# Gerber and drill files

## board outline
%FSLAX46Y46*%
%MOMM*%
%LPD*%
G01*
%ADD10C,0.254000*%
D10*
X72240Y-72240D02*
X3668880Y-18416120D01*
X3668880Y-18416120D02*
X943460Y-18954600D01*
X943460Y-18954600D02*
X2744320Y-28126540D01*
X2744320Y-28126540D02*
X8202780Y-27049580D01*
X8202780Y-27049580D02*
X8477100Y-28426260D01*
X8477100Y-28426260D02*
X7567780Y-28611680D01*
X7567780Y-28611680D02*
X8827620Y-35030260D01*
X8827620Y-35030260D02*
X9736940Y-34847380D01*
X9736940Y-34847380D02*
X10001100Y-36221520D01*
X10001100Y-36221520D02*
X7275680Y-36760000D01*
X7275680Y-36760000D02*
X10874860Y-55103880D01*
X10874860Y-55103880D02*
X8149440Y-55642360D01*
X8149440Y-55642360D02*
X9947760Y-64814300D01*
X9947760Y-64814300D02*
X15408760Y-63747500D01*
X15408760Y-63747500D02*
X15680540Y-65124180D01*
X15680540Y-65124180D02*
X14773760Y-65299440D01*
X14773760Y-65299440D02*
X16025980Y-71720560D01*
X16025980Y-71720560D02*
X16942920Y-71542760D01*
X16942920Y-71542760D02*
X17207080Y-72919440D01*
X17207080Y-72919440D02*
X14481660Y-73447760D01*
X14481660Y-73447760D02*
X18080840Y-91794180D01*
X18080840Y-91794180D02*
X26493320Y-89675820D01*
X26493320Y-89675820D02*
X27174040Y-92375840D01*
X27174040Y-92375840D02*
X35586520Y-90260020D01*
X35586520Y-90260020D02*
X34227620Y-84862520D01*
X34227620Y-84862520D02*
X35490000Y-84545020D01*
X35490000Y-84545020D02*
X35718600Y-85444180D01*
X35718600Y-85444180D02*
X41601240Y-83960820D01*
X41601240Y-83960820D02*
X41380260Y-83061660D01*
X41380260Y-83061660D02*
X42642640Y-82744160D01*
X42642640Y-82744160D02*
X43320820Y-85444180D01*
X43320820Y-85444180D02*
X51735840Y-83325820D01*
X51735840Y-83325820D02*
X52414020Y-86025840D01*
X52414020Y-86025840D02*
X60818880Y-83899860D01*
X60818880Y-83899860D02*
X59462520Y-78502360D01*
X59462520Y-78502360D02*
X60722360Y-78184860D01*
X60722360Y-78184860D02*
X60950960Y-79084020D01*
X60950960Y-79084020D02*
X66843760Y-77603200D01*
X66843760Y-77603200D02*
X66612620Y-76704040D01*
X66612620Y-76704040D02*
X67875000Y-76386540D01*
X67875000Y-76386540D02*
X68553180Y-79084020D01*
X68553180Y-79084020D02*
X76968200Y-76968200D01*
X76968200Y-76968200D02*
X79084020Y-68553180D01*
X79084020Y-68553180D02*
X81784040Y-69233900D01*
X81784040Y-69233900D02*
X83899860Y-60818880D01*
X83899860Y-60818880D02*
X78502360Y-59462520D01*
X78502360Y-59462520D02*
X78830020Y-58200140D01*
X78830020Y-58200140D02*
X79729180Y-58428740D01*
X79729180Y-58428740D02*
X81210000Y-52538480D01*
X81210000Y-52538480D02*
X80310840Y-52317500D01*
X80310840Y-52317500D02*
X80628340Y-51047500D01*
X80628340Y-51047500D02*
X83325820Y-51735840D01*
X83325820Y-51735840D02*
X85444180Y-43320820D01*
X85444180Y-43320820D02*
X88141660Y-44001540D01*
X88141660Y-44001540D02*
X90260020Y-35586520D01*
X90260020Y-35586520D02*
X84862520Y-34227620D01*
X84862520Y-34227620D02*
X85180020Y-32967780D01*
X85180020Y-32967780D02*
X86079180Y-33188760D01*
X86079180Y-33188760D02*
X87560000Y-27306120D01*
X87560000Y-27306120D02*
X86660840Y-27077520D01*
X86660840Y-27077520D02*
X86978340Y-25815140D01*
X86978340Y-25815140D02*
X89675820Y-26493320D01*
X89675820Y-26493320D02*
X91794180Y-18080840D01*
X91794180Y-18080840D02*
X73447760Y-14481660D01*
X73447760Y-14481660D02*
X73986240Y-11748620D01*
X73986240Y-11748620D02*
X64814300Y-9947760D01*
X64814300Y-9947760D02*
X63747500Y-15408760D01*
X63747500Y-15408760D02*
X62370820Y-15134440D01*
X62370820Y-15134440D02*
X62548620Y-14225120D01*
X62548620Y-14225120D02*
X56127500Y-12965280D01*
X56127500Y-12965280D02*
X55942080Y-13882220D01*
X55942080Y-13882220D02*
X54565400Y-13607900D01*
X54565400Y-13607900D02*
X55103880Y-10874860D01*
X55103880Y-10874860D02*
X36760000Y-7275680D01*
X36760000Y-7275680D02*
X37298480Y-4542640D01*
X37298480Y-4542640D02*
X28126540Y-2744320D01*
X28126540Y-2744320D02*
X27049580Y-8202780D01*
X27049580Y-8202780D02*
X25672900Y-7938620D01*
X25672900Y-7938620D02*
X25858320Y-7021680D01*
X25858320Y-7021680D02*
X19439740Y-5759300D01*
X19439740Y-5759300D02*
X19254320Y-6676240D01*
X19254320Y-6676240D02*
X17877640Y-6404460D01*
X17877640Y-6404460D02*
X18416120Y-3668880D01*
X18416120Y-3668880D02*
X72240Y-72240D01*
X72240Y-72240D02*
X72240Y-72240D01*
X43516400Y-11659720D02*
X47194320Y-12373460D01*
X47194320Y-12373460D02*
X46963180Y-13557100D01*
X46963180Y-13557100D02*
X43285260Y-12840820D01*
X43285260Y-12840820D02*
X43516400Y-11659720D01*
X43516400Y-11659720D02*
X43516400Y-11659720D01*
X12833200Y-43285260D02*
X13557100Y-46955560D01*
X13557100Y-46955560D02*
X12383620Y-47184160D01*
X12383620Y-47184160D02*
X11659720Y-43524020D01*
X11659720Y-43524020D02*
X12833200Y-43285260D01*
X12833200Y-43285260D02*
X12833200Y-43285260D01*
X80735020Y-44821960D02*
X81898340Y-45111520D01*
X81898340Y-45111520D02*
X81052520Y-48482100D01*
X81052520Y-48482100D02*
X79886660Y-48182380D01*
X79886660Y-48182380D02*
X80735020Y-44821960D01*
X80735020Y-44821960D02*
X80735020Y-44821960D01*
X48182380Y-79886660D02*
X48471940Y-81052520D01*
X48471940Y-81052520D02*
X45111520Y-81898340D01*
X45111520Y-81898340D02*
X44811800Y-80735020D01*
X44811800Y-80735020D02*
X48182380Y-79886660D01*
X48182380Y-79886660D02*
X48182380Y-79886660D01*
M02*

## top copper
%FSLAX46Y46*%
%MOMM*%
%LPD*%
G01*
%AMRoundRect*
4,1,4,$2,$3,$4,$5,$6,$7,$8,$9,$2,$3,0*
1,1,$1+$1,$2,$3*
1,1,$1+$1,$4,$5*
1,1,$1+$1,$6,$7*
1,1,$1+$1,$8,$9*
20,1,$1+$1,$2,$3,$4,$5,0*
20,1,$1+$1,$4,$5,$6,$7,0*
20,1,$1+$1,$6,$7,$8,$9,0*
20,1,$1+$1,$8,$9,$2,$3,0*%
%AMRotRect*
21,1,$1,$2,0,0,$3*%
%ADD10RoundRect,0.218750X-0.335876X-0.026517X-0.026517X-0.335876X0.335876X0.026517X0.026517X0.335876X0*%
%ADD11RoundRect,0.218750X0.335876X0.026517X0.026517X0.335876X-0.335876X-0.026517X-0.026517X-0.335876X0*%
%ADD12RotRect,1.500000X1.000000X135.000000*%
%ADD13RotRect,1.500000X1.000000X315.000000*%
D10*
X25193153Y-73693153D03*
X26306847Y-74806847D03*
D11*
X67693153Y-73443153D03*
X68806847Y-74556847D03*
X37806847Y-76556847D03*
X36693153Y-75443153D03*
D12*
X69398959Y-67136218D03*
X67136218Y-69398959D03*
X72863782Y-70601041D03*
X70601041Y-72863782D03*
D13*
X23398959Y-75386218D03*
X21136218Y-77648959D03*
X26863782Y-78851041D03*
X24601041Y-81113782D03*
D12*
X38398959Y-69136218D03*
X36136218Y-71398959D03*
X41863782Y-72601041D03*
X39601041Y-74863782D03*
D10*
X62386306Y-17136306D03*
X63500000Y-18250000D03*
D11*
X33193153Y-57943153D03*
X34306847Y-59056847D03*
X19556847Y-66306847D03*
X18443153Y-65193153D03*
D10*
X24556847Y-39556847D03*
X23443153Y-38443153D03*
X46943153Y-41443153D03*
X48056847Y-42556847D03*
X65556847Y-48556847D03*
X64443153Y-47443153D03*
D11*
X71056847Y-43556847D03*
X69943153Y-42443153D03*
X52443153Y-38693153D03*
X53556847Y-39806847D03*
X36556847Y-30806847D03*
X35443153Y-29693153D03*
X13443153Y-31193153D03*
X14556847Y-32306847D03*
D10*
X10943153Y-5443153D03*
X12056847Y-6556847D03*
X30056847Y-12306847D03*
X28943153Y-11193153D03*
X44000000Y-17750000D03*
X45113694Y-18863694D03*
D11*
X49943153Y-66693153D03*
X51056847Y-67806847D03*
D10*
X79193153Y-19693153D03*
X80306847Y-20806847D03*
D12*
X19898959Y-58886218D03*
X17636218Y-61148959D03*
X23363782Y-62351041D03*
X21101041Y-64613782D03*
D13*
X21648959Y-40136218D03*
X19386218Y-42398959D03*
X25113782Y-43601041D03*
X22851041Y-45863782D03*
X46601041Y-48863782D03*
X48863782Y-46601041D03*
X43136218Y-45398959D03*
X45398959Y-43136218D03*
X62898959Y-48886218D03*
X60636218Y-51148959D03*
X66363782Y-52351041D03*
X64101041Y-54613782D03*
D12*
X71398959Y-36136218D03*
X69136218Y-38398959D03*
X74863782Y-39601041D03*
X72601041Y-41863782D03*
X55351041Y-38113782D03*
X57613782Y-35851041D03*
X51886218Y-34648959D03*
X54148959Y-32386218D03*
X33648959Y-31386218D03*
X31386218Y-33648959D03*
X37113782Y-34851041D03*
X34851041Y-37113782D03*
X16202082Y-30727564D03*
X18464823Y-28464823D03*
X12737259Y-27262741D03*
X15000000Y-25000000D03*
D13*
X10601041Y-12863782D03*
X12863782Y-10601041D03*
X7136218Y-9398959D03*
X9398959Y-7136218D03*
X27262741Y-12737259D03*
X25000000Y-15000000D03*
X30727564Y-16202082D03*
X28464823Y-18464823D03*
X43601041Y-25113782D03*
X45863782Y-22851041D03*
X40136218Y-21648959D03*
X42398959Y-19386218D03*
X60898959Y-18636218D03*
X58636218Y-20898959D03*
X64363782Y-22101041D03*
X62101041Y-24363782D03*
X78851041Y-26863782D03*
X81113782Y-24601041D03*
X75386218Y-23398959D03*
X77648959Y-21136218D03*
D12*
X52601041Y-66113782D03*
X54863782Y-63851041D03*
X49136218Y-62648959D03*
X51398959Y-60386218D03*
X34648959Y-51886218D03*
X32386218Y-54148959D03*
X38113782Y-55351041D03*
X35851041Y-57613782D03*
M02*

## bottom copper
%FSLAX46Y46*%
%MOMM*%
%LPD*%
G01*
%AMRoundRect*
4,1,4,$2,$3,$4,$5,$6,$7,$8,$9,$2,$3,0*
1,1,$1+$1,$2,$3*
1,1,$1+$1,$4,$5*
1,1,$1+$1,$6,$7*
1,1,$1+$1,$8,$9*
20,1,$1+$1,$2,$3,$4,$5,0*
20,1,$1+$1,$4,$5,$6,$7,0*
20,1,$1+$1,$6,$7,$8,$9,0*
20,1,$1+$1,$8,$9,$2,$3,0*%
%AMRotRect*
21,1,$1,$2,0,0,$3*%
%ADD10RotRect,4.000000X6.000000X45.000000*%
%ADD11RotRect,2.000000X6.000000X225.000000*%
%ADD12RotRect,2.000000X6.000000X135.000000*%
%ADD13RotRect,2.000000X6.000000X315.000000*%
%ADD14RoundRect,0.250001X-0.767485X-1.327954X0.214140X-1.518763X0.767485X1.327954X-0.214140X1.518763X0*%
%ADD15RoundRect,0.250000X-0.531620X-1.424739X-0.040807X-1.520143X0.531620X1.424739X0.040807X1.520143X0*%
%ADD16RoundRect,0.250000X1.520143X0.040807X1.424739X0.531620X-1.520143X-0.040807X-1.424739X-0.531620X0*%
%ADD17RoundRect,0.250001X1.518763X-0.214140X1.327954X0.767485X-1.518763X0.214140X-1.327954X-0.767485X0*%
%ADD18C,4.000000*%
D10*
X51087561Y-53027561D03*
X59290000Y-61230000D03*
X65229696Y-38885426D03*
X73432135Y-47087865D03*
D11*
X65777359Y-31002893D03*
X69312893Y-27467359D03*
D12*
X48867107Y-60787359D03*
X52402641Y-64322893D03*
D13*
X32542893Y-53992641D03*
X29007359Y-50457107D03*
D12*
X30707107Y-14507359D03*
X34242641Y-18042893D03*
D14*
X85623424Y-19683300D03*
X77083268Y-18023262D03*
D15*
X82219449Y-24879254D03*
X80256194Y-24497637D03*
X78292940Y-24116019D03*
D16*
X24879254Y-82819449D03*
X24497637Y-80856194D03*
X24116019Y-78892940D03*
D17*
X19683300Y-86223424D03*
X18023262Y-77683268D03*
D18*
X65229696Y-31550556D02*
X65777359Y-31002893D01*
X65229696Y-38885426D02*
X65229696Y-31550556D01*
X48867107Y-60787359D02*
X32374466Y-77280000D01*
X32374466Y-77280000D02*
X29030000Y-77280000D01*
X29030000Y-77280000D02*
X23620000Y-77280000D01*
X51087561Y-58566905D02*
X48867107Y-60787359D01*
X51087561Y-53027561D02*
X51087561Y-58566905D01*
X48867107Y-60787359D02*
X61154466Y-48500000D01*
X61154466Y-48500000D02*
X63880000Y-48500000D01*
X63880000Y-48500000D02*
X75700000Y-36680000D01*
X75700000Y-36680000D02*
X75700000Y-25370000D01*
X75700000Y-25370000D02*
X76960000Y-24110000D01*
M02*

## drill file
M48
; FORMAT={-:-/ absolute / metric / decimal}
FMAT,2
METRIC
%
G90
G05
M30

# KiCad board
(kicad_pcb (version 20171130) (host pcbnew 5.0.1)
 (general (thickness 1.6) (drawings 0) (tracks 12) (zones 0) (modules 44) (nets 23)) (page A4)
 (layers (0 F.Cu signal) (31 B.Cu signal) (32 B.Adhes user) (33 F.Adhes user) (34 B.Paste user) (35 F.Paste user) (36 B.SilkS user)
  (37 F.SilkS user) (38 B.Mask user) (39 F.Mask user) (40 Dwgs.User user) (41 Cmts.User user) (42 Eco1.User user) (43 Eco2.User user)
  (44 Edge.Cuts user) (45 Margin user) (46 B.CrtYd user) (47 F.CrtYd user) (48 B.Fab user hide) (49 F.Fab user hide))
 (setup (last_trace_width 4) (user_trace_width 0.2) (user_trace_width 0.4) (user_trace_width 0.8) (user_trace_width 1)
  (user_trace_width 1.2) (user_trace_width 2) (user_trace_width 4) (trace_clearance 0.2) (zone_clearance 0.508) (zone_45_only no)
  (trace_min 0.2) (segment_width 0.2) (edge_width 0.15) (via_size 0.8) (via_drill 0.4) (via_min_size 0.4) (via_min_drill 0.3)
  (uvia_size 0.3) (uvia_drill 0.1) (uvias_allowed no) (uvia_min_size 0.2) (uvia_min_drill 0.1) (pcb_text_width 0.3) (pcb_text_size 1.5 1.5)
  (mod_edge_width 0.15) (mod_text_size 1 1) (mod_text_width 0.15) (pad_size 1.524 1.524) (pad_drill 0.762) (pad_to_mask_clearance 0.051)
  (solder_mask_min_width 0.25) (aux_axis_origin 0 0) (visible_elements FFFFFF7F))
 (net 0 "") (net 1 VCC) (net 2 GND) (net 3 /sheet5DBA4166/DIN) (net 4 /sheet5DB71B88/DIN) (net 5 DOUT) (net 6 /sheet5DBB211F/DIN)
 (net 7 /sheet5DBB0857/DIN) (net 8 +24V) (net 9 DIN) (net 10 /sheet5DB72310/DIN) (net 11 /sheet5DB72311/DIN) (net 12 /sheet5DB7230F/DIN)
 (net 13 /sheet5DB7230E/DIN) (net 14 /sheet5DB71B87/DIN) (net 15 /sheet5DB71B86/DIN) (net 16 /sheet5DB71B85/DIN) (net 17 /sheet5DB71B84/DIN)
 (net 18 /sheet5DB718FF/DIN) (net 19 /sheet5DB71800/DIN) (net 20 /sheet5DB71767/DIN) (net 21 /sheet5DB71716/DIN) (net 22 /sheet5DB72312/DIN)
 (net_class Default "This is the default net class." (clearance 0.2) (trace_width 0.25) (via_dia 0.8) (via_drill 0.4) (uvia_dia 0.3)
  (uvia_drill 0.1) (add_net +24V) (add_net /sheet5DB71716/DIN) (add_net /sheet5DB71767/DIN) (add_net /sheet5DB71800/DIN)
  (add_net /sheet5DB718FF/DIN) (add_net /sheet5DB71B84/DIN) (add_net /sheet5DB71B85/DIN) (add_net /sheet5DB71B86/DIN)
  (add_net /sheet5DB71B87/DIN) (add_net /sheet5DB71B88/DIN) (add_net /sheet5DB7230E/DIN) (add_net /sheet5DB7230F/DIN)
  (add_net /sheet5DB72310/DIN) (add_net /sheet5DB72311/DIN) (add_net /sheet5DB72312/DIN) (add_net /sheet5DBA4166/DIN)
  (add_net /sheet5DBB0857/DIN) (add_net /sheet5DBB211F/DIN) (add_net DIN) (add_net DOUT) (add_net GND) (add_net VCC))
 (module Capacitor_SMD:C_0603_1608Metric (layer F.Cu) (at 25.75 74.25 315)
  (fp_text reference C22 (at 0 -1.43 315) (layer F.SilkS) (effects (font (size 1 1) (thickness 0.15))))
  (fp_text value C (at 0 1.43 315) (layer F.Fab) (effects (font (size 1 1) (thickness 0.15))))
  (pad 1 smd roundrect (at -0.7875 0 315) (size 0.875 0.95) (layers F.Cu F.Paste F.Mask) (roundrect_rratio 0.25) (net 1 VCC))
  (pad 2 smd roundrect (at 0.7875 0 315) (size 0.875 0.95) (layers F.Cu F.Paste F.Mask) (roundrect_rratio 0.25) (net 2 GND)))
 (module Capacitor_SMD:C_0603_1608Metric (layer F.Cu) (at 68.25 74 135)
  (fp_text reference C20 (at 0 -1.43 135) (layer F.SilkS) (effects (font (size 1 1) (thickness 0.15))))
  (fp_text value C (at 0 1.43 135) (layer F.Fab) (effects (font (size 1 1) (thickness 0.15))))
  (pad 2 smd roundrect (at 0.7875 0 135) (size 0.875 0.95) (layers F.Cu F.Paste F.Mask) (roundrect_rratio 0.25) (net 2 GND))
  (pad 1 smd roundrect (at -0.7875 0 135) (size 0.875 0.95) (layers F.Cu F.Paste F.Mask) (roundrect_rratio 0.25) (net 1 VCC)))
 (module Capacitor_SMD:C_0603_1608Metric (layer F.Cu) (at 37.25 76 135)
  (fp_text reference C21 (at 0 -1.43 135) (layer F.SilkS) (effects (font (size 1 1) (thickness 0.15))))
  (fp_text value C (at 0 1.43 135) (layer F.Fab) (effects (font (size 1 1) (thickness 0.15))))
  (pad 1 smd roundrect (at -0.7875 0 135) (size 0.875 0.95) (layers F.Cu F.Paste F.Mask) (roundrect_rratio 0.25) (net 1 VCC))
  (pad 2 smd roundrect (at 0.7875 0 135) (size 0.875 0.95) (layers F.Cu F.Paste F.Mask) (roundrect_rratio 0.25) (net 2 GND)))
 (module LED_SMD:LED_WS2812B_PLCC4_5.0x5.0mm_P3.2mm (layer F.Cu) (at 70 70 135)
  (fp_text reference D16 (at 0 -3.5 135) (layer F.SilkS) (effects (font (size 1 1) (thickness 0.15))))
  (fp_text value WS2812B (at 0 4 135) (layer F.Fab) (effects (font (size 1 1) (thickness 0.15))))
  (pad 3 smd rect (at 2.45 1.6 135) (size 1.5 1) (layers F.Cu F.Paste F.Mask) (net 2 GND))
  (pad 4 smd rect (at 2.45 -1.6 135) (size 1.5 1) (layers F.Cu F.Paste F.Mask) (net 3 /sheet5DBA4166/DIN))
  (pad 2 smd rect (at -2.45 1.6 135) (size 1.5 1) (layers F.Cu F.Paste F.Mask) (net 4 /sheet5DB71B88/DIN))
  (pad 1 smd rect (at -2.45 -1.6 135) (size 1.5 1) (layers F.Cu F.Paste F.Mask) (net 1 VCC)))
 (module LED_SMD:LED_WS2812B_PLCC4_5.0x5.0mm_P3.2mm (layer F.Cu) (at 24 78.25 315)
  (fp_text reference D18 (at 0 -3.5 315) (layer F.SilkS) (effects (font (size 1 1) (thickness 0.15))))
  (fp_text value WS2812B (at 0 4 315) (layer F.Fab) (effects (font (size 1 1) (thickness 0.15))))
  (pad 1 smd rect (at -2.45 -1.6 315) (size 1.5 1) (layers F.Cu F.Paste F.Mask) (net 1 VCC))
  (pad 2 smd rect (at -2.45 1.6 315) (size 1.5 1) (layers F.Cu F.Paste F.Mask) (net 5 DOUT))
  (pad 4 smd rect (at 2.45 -1.6 315) (size 1.5 1) (layers F.Cu F.Paste F.Mask) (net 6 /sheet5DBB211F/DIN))
  (pad 3 smd rect (at 2.45 1.6 315) (size 1.5 1) (layers F.Cu F.Paste F.Mask) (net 2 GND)))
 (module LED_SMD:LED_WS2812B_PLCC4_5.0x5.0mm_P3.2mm (layer F.Cu) (at 39 72 135)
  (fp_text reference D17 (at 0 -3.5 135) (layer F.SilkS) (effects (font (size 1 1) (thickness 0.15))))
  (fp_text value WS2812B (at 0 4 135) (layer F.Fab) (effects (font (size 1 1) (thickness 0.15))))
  (pad 3 smd rect (at 2.45 1.6 135) (size 1.5 1) (layers F.Cu F.Paste F.Mask) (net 2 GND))
  (pad 4 smd rect (at 2.45 -1.6 135) (size 1.5 1) (layers F.Cu F.Paste F.Mask) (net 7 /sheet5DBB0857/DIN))
  (pad 2 smd rect (at -2.45 1.6 135) (size 1.5 1) (layers F.Cu F.Paste F.Mask) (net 6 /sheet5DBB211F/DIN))
  (pad 1 smd rect (at -2.45 -1.6 135) (size 1.5 1) (layers F.Cu F.Paste F.Mask) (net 1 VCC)))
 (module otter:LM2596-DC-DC (layer B.Cu) (at 62.259848 50.057713 45)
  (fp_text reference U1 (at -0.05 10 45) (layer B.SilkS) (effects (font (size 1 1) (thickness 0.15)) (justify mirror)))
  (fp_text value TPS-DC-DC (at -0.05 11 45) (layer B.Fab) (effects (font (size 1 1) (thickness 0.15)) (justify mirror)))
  (pad 1 smd rect (at -10 -5.8 45) (size 4 6) (layers B.Cu B.Paste B.Mask) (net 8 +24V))
  (pad 2 smd rect (at -10 5.8 45) (size 4 6) (layers B.Cu B.Paste B.Mask) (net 2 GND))
  (pad 4 smd rect (at 10 -5.8 45) (size 4 6) (layers B.Cu B.Paste B.Mask) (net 1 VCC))
  (pad 3 smd rect (at 10 5.8 45) (size 4 6) (layers B.Cu B.Paste B.Mask) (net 2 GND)))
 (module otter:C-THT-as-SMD (layer B.Cu) (at 70.02 31.71 225)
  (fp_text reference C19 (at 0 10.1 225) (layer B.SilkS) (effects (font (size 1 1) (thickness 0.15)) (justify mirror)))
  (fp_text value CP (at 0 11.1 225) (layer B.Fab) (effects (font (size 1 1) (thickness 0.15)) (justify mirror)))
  (pad 1 smd rect (at 2.5 3.5 225) (size 2 6) (layers B.Cu B.Paste B.Mask) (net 1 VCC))
  (pad 2 smd rect (at -2.5 3.5 225) (size 2 6) (layers B.Cu B.Paste B.Mask) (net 2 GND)))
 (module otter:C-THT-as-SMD (layer B.Cu) (at 48.16 65.03 135)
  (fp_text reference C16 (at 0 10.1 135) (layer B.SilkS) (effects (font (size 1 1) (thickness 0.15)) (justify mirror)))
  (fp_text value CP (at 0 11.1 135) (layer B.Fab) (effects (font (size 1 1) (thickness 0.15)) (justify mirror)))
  (pad 1 smd rect (at 2.5 3.5 135) (size 2 6) (layers B.Cu B.Paste B.Mask) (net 8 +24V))
  (pad 2 smd rect (at -2.5 3.5 135) (size 2 6) (layers B.Cu B.Paste B.Mask) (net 2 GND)))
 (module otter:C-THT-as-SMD (layer B.Cu) (at 33.25 49.75 315)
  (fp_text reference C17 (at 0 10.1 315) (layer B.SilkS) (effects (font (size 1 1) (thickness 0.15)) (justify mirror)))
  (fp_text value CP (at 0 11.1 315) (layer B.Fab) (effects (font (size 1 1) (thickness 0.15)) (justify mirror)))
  (pad 1 smd rect (at 2.5 3.5 315) (size 2 6) (layers B.Cu B.Paste B.Mask) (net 1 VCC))
  (pad 2 smd rect (at -2.5 3.5 315) (size 2 6) (layers B.Cu B.Paste B.Mask) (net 2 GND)))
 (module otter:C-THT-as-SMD (layer B.Cu) (at 30 18.75 135)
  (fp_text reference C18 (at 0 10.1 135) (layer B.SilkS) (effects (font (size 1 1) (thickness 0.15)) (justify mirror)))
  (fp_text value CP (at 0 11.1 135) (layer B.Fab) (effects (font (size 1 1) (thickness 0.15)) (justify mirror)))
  (pad 1 smd rect (at 2.5 3.5 135) (size 2 6) (layers B.Cu B.Paste B.Mask) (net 1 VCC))
  (pad 2 smd rect (at -2.5 3.5 135) (size 2 6) (layers B.Cu B.Paste B.Mask) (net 2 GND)))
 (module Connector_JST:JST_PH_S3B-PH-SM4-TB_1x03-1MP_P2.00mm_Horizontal (layer B.Cu) (at 80.8 21.7 349)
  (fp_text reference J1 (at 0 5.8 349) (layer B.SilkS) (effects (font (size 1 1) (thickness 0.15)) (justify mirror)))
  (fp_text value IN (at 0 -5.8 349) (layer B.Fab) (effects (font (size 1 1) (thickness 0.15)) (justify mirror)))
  (pad MP smd roundrect (at 4.35 -2.9 349) (size 1.5 3.4) (layers B.Cu B.Paste B.Mask) (roundrect_rratio 0.166667) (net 2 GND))
  (pad MP smd roundrect (at -4.35 -2.9 349) (size 1.5 3.4) (layers B.Cu B.Paste B.Mask) (roundrect_rratio 0.166667) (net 2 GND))
  (pad 3 smd roundrect (at 2 2.849999 349) (size 1 3.5) (layers B.Cu B.Paste B.Mask) (roundrect_rratio 0.25) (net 2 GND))
  (pad 2 smd roundrect (at 0 2.85 349) (size 1 3.5) (layers B.Cu B.Paste B.Mask) (roundrect_rratio 0.25) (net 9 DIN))
  (pad 1 smd roundrect (at -2 2.85 349) (size 1 3.5) (layers B.Cu B.Paste B.Mask) (roundrect_rratio 0.25) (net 8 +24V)))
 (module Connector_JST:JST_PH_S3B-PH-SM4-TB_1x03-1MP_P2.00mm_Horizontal (layer B.Cu) (at 21.7 81.4 101)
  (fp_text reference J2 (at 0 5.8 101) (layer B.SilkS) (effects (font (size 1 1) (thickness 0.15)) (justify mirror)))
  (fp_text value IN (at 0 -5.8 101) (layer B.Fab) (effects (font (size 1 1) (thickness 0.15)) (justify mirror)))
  (pad 1 smd roundrect (at -2 2.849999 101) (size 1 3.5) (layers B.Cu B.Paste B.Mask) (roundrect_rratio 0.25) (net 2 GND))
  (pad 2 smd roundrect (at 0 2.85 101) (size 1 3.5) (layers B.Cu B.Paste B.Mask) (roundrect_rratio 0.25) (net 5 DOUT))
  (pad 3 smd roundrect (at 2 2.85 101) (size 1 3.5) (layers B.Cu B.Paste B.Mask) (roundrect_rratio 0.25) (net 8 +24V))
  (pad MP smd roundrect (at -4.35 -2.9 101) (size 1.5 3.4) (layers B.Cu B.Paste B.Mask) (roundrect_rratio 0.166667) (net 2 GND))
  (pad MP smd roundrect (at 4.35 -2.9 101) (size 1.5 3.4) (layers B.Cu B.Paste B.Mask) (roundrect_rratio 0.166667) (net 2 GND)))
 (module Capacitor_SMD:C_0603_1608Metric (layer F.Cu) (at 62.943153 17.693153 315)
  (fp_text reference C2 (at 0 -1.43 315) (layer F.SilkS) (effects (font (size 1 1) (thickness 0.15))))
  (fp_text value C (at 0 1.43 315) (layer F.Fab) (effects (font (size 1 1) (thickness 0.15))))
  (pad 1 smd roundrect (at -0.7875 0 315) (size 0.875 0.95) (layers F.Cu F.Paste F.Mask) (roundrect_rratio 0.25) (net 1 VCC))
  (pad 2 smd roundrect (at 0.7875 0 315) (size 0.875 0.95) (layers F.Cu F.Paste F.Mask) (roundrect_rratio 0.25) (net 2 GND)))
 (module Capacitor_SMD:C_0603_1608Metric (layer F.Cu) (at 33.75 58.5 135)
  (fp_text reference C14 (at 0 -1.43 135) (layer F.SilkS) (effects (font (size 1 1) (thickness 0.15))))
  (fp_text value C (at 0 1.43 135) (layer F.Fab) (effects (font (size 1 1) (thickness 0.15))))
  (pad 2 smd roundrect (at 0.7875 0 135) (size 0.875 0.95) (layers F.Cu F.Paste F.Mask) (roundrect_rratio 0.25) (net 2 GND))
  (pad 1 smd roundrect (at -0.7875 0 135) (size 0.875 0.95) (layers F.Cu F.Paste F.Mask) (roundrect_rratio 0.25) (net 1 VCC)))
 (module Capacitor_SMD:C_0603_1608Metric (layer F.Cu) (at 19 65.75 135)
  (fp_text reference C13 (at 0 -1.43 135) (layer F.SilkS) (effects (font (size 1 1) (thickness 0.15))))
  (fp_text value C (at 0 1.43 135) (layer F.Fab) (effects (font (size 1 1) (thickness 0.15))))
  (pad 1 smd roundrect (at -0.7875 0 135) (size 0.875 0.95) (layers F.Cu F.Paste F.Mask) (roundrect_rratio 0.25) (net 1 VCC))
  (pad 2 smd roundrect (at 0.7875 0 135) (size 0.875 0.95) (layers F.Cu F.Paste F.Mask) (roundrect_rratio 0.25) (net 2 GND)))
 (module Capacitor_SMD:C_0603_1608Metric (layer F.Cu) (at 24 39 315)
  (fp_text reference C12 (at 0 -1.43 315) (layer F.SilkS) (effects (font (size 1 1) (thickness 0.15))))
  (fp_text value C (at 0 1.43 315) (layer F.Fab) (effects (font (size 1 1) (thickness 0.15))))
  (pad 2 smd roundrect (at 0.7875 0 315) (size 0.875 0.95) (layers F.Cu F.Paste F.Mask) (roundrect_rratio 0.25) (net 2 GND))
  (pad 1 smd roundrect (at -0.7875 0 315) (size 0.875 0.95) (layers F.Cu F.Paste F.Mask) (roundrect_rratio 0.25) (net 1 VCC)))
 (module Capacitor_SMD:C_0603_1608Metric (layer F.Cu) (at 47.5 42 315)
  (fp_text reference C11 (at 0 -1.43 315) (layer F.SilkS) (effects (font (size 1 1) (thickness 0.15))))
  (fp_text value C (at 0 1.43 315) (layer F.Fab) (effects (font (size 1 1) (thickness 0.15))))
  (pad 1 smd roundrect (at -0.7875 0 315) (size 0.875 0.95) (layers F.Cu F.Paste F.Mask) (roundrect_rratio 0.25) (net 1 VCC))
  (pad 2 smd roundrect (at 0.7875 0 315) (size 0.875 0.95) (layers F.Cu F.Paste F.Mask) (roundrect_rratio 0.25) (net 2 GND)))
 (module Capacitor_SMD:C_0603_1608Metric (layer F.Cu) (at 65 48 315)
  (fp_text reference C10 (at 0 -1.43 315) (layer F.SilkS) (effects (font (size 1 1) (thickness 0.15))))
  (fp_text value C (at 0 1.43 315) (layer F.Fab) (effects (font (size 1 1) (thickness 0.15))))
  (pad 2 smd roundrect (at 0.7875 0 315) (size 0.875 0.95) (layers F.Cu F.Paste F.Mask) (roundrect_rratio 0.25) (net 2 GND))
  (pad 1 smd roundrect (at -0.7875 0 315) (size 0.875 0.95) (layers F.Cu F.Paste F.Mask) (roundrect_rratio 0.25) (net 1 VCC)))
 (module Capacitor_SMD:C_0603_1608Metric (layer F.Cu) (at 70.5 43 135)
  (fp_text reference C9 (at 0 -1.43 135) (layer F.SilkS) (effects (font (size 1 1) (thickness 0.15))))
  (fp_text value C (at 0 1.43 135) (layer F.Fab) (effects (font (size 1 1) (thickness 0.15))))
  (pad 1 smd roundrect (at -0.7875 0 135) (size 0.875 0.95) (layers F.Cu F.Paste F.Mask) (roundrect_rratio 0.25) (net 1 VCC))
  (pad 2 smd roundrect (at 0.7875 0 135) (size 0.875 0.95) (layers F.Cu F.Paste F.Mask) (roundrect_rratio 0.25) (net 2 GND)))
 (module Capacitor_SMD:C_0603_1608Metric (layer F.Cu) (at 53 39.25 135)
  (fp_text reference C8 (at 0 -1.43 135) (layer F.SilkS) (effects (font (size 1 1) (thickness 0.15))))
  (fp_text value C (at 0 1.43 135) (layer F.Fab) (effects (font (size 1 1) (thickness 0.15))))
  (pad 2 smd roundrect (at 0.7875 0 135) (size 0.875 0.95) (layers F.Cu F.Paste F.Mask) (roundrect_rratio 0.25) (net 2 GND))
  (pad 1 smd roundrect (at -0.7875 0 135) (size 0.875 0.95) (layers F.Cu F.Paste F.Mask) (roundrect_rratio 0.25) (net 1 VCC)))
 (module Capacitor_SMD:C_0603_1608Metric (layer F.Cu) (at 36 30.25 135)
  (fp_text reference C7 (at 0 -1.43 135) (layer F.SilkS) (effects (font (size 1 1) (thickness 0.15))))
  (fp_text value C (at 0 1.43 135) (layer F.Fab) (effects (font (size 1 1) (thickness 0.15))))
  (pad 1 smd roundrect (at -0.7875 0 135) (size 0.875 0.95) (layers F.Cu F.Paste F.Mask) (roundrect_rratio 0.25) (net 1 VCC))
  (pad 2 smd roundrect (at 0.7875 0 135) (size 0.875 0.95) (layers F.Cu F.Paste F.Mask) (roundrect_rratio 0.25) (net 2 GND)))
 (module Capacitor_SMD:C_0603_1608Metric (layer F.Cu) (at 14 31.75 135)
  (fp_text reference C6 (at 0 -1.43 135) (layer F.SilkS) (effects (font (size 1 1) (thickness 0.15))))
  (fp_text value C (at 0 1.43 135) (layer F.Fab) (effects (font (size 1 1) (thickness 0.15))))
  (pad 2 smd roundrect (at 0.7875 0 135) (size 0.875 0.95) (layers F.Cu F.Paste F.Mask) (roundrect_rratio 0.25) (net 2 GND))
  (pad 1 smd roundrect (at -0.7875 0 135) (size 0.875 0.95) (layers F.Cu F.Paste F.Mask) (roundrect_rratio 0.25) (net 1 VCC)))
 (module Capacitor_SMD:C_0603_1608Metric (layer F.Cu) (at 11.5 6 315)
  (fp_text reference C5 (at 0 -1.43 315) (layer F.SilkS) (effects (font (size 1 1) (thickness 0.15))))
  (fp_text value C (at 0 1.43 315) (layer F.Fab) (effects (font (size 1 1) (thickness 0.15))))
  (pad 1 smd roundrect (at -0.7875 0 315) (size 0.875 0.95) (layers F.Cu F.Paste F.Mask) (roundrect_rratio 0.25) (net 1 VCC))
  (pad 2 smd roundrect (at 0.7875 0 315) (size 0.875 0.95) (layers F.Cu F.Paste F.Mask) (roundrect_rratio 0.25) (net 2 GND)))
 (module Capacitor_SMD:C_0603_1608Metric (layer F.Cu) (at 29.5 11.75 315)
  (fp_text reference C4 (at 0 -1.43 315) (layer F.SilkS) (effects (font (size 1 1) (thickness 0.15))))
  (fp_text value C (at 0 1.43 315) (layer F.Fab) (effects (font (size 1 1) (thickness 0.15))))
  (pad 2 smd roundrect (at 0.7875 0 315) (size 0.875 0.95) (layers F.Cu F.Paste F.Mask) (roundrect_rratio 0.25) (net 2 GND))
  (pad 1 smd roundrect (at -0.7875 0 315) (size 0.875 0.95) (layers F.Cu F.Paste F.Mask) (roundrect_rratio 0.25) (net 1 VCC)))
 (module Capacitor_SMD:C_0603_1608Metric (layer F.Cu) (at 44.556847 18.306847 315)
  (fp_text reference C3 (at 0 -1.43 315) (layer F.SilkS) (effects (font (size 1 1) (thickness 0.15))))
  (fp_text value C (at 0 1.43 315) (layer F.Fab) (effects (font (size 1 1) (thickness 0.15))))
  (pad 1 smd roundrect (at -0.7875 0 315) (size 0.875 0.95) (layers F.Cu F.Paste F.Mask) (roundrect_rratio 0.25) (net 1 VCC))
  (pad 2 smd roundrect (at 0.7875 0 315) (size 0.875 0.95) (layers F.Cu F.Paste F.Mask) (roundrect_rratio 0.25) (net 2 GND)))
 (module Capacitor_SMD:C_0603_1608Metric (layer F.Cu) (at 50.5 67.25 135)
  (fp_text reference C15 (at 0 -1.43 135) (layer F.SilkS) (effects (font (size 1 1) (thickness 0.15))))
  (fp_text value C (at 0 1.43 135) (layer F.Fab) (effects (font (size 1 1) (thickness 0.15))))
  (pad 2 smd roundrect (at 0.7875 0 135) (size 0.875 0.95) (layers F.Cu F.Paste F.Mask) (roundrect_rratio 0.25) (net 2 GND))
  (pad 1 smd roundrect (at -0.7875 0 135) (size 0.875 0.95) (layers F.Cu F.Paste F.Mask) (roundrect_rratio 0.25) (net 1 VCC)))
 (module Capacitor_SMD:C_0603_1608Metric (layer F.Cu) (at 79.75 20.25 315)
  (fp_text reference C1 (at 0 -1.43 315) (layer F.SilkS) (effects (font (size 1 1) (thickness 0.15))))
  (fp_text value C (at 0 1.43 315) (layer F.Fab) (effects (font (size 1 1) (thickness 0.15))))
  (pad 1 smd roundrect (at -0.7875 0 315) (size 0.875 0.95) (layers F.Cu F.Paste F.Mask) (roundrect_rratio 0.25) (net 1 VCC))
  (pad 2 smd roundrect (at 0.7875 0 315) (size 0.875 0.95) (layers F.Cu F.Paste F.Mask) (roundrect_rratio 0.25) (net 2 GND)))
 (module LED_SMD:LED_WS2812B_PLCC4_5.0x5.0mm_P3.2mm (layer F.Cu) (at 20.5 61.75 135)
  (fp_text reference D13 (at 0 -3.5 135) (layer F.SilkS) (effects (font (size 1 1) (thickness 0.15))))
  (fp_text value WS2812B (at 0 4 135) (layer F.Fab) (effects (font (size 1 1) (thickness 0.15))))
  (pad 3 smd rect (at 2.45 1.6 135) (size 1.5 1) (layers F.Cu F.Paste F.Mask) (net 2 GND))
  (pad 4 smd rect (at 2.45 -1.6 135) (size 1.5 1) (layers F.Cu F.Paste F.Mask) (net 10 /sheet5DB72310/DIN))
  (pad 2 smd rect (at -2.45 1.6 135) (size 1.5 1) (layers F.Cu F.Paste F.Mask) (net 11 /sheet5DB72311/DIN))
  (pad 1 smd rect (at -2.45 -1.6 135) (size 1.5 1) (layers F.Cu F.Paste F.Mask) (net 1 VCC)))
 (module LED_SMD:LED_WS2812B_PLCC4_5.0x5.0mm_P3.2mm (layer F.Cu) (at 22.25 43 315)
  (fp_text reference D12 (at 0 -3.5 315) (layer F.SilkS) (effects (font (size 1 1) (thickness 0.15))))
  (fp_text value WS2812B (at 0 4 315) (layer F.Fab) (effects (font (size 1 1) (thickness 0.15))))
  (pad 1 smd rect (at -2.45 -1.6 315) (size 1.5 1) (layers F.Cu F.Paste F.Mask) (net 1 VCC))
  (pad 2 smd rect (at -2.45 1.6 315) (size 1.5 1) (layers F.Cu F.Paste F.Mask) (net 10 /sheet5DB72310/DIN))
  (pad 4 smd rect (at 2.45 -1.6 315) (size 1.5 1) (layers F.Cu F.Paste F.Mask) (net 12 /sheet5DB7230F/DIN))
  (pad 3 smd rect (at 2.45 1.6 315) (size 1.5 1) (layers F.Cu F.Paste F.Mask) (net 2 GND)))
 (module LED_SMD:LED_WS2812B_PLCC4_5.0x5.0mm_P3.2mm (layer F.Cu) (at 46 46 315)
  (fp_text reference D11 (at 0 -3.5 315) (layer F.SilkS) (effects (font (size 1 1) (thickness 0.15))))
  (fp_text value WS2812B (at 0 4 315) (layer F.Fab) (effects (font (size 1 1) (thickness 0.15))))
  (pad 3 smd rect (at 2.45 1.6 315) (size 1.5 1) (layers F.Cu F.Paste F.Mask) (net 2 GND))
  (pad 4 smd rect (at 2.45 -1.6 315) (size 1.5 1) (layers F.Cu F.Paste F.Mask) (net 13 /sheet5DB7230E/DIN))
  (pad 2 smd rect (at -2.45 1.6 315) (size 1.5 1) (layers F.Cu F.Paste F.Mask) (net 12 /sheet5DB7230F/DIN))
  (pad 1 smd rect (at -2.45 -1.6 315) (size 1.5 1) (layers F.Cu F.Paste F.Mask) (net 1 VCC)))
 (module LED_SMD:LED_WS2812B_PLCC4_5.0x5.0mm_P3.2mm (layer F.Cu) (at 63.5 51.75 315)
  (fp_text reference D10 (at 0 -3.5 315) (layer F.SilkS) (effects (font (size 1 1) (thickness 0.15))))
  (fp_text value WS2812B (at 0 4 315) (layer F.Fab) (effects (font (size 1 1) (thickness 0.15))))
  (pad 1 smd rect (at -2.45 -1.6 315) (size 1.5 1) (layers F.Cu F.Paste F.Mask) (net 1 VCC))
  (pad 2 smd rect (at -2.45 1.6 315) (size 1.5 1) (layers F.Cu F.Paste F.Mask) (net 13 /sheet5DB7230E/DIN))
  (pad 4 smd rect (at 2.45 -1.6 315) (size 1.5 1) (layers F.Cu F.Paste F.Mask) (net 4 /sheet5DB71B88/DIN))
  (pad 3 smd rect (at 2.45 1.6 315) (size 1.5 1) (layers F.Cu F.Paste F.Mask) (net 2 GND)))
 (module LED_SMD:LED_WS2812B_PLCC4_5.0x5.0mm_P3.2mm (layer F.Cu) (at 72 39 135)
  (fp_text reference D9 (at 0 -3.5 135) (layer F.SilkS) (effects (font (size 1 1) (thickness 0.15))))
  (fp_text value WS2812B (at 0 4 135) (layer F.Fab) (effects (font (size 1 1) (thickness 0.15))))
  (pad 3 smd rect (at 2.45 1.6 135) (size 1.5 1) (layers F.Cu F.Paste F.Mask) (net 2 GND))
  (pad 4 smd rect (at 2.45 -1.6 135) (size 1.5 1) (layers F.Cu F.Paste F.Mask) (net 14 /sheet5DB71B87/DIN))
  (pad 2 smd rect (at -2.45 1.6 135) (size 1.5 1) (layers F.Cu F.Paste F.Mask) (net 3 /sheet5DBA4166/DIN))
  (pad 1 smd rect (at -2.45 -1.6 135) (size 1.5 1) (layers F.Cu F.Paste F.Mask) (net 1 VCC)))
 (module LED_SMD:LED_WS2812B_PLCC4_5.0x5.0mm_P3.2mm (layer F.Cu) (at 54.75 35.25 135)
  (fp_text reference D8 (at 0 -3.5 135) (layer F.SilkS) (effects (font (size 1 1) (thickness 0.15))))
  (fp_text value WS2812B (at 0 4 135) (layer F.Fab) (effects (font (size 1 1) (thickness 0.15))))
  (pad 1 smd rect (at -2.45 -1.6 135) (size 1.5 1) (layers F.Cu F.Paste F.Mask) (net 1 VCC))
  (pad 2 smd rect (at -2.45 1.6 135) (size 1.5 1) (layers F.Cu F.Paste F.Mask) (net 14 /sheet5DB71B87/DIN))
  (pad 4 smd rect (at 2.45 -1.6 135) (size 1.5 1) (layers F.Cu F.Paste F.Mask) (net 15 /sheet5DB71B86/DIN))
  (pad 3 smd rect (at 2.45 1.6 135) (size 1.5 1) (layers F.Cu F.Paste F.Mask) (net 2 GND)))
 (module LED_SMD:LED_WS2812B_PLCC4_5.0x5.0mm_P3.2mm (layer F.Cu) (at 34.25 34.25 135)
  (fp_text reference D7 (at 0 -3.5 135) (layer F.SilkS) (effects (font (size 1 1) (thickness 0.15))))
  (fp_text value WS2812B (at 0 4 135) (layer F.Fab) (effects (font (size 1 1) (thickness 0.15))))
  (pad 3 smd rect (at 2.45 1.6 135) (size 1.5 1) (layers F.Cu F.Paste F.Mask) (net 2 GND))
  (pad 4 smd rect (at 2.45 -1.6 135) (size 1.5 1) (layers F.Cu F.Paste F.Mask) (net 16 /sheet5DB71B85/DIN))
  (pad 2 smd rect (at -2.45 1.6 135) (size 1.5 1) (layers F.Cu F.Paste F.Mask) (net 15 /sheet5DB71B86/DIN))
  (pad 1 smd rect (at -2.45 -1.6 135) (size 1.5 1) (layers F.Cu F.Paste F.Mask) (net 1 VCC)))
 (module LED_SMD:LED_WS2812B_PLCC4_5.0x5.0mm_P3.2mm (layer F.Cu) (at 15.601041 27.863782 135)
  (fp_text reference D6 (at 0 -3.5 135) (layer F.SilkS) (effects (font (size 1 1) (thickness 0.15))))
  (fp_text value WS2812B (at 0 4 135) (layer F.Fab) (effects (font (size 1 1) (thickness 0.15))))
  (pad 1 smd rect (at -2.45 -1.6 135) (size 1.5 1) (layers F.Cu F.Paste F.Mask) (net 1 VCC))
  (pad 2 smd rect (at -2.45 1.6 135) (size 1.5 1) (layers F.Cu F.Paste F.Mask) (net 16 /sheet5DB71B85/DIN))
  (pad 4 smd rect (at 2.45 -1.6 135) (size 1.5 1) (layers F.Cu F.Paste F.Mask) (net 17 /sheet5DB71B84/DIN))
  (pad 3 smd rect (at 2.45 1.6 135) (size 1.5 1) (layers F.Cu F.Paste F.Mask) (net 2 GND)))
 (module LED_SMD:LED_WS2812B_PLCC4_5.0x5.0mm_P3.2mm (layer F.Cu) (at 10 10 315)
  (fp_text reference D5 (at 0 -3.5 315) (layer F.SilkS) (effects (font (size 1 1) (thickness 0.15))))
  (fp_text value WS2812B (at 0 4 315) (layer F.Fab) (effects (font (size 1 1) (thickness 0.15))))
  (pad 3 smd rect (at 2.45 1.6 315) (size 1.5 1) (layers F.Cu F.Paste F.Mask) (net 2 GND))
  (pad 4 smd rect (at 2.45 -1.6 315) (size 1.5 1) (layers F.Cu F.Paste F.Mask) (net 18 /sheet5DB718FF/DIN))
  (pad 2 smd rect (at -2.45 1.6 315) (size 1.5 1) (layers F.Cu F.Paste F.Mask) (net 17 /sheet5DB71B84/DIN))
  (pad 1 smd rect (at -2.45 -1.6 315) (size 1.5 1) (layers F.Cu F.Paste F.Mask) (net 1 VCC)))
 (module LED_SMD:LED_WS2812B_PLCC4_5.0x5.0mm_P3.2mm (layer F.Cu) (at 27.863782 15.601041 315)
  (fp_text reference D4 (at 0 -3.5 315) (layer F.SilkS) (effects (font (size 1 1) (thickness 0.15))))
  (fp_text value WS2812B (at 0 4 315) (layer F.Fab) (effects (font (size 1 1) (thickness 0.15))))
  (pad 1 smd rect (at -2.45 -1.6 315) (size 1.5 1) (layers F.Cu F.Paste F.Mask) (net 1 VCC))
  (pad 2 smd rect (at -2.45 1.6 315) (size 1.5 1) (layers F.Cu F.Paste F.Mask) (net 18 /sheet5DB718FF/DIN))
  (pad 4 smd rect (at 2.45 -1.6 315) (size 1.5 1) (layers F.Cu F.Paste F.Mask) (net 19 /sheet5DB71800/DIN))
  (pad 3 smd rect (at 2.45 1.6 315) (size 1.5 1) (layers F.Cu F.Paste F.Mask) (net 2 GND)))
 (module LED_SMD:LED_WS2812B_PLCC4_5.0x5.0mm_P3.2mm (layer F.Cu) (at 43 22.25 315)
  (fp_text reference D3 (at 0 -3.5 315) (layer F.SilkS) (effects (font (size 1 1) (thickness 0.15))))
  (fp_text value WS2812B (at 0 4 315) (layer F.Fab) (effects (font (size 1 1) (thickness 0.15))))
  (pad 3 smd rect (at 2.45 1.6 315) (size 1.5 1) (layers F.Cu F.Paste F.Mask) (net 2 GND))
  (pad 4 smd rect (at 2.45 -1.6 315) (size 1.5 1) (layers F.Cu F.Paste F.Mask) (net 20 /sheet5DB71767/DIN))
  (pad 2 smd rect (at -2.45 1.6 315) (size 1.5 1) (layers F.Cu F.Paste F.Mask) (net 19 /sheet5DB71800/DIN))
  (pad 1 smd rect (at -2.45 -1.6 315) (size 1.5 1) (layers F.Cu F.Paste F.Mask) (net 1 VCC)))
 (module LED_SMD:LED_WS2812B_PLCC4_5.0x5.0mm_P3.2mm (layer F.Cu) (at 61.5 21.5 315)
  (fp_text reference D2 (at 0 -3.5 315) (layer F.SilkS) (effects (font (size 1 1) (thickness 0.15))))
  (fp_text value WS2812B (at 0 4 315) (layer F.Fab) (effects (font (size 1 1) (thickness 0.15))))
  (pad 1 smd rect (at -2.45 -1.6 315) (size 1.5 1) (layers F.Cu F.Paste F.Mask) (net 1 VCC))
  (pad 2 smd rect (at -2.45 1.6 315) (size 1.5 1) (layers F.Cu F.Paste F.Mask) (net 20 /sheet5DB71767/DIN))
  (pad 4 smd rect (at 2.45 -1.6 315) (size 1.5 1) (layers F.Cu F.Paste F.Mask) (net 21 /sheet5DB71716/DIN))
  (pad 3 smd rect (at 2.45 1.6 315) (size 1.5 1) (layers F.Cu F.Paste F.Mask) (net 2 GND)))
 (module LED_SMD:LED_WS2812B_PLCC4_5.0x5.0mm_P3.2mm (layer F.Cu) (at 78.25 24 315)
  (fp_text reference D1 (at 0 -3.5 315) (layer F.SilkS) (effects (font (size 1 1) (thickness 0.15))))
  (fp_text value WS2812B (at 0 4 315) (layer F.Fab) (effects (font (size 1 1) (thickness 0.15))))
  (pad 3 smd rect (at 2.45 1.6 315) (size 1.5 1) (layers F.Cu F.Paste F.Mask) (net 2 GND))
  (pad 4 smd rect (at 2.45 -1.6 315) (size 1.5 1) (layers F.Cu F.Paste F.Mask) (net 9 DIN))
  (pad 2 smd rect (at -2.45 1.6 315) (size 1.5 1) (layers F.Cu F.Paste F.Mask) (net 21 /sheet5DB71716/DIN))
  (pad 1 smd rect (at -2.45 -1.6 315) (size 1.5 1) (layers F.Cu F.Paste F.Mask) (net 1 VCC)))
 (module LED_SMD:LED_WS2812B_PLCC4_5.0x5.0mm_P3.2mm (layer F.Cu) (at 52 63.25 135)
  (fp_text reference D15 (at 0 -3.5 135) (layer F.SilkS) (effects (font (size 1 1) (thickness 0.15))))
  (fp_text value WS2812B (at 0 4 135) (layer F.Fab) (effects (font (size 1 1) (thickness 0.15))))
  (pad 1 smd rect (at -2.45 -1.6 135) (size 1.5 1) (layers F.Cu F.Paste F.Mask) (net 1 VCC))
  (pad 2 smd rect (at -2.45 1.6 135) (size 1.5 1) (layers F.Cu F.Paste F.Mask) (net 7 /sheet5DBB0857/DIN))
  (pad 4 smd rect (at 2.45 -1.6 135) (size 1.5 1) (layers F.Cu F.Paste F.Mask) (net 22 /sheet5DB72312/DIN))
  (pad 3 smd rect (at 2.45 1.6 135) (size 1.5 1) (layers F.Cu F.Paste F.Mask) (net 2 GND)))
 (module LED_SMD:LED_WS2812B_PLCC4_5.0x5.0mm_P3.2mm (layer F.Cu) (at 35.25 54.75 135)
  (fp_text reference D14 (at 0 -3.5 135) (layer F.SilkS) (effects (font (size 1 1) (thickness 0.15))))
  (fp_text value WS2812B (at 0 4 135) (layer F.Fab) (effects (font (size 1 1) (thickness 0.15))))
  (pad 3 smd rect (at 2.45 1.6 135) (size 1.5 1) (layers F.Cu F.Paste F.Mask) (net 2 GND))
  (pad 4 smd rect (at 2.45 -1.6 135) (size 1.5 1) (layers F.Cu F.Paste F.Mask) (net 11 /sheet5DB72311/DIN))
  (pad 2 smd rect (at -2.45 1.6 135) (size 1.5 1) (layers F.Cu F.Paste F.Mask) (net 22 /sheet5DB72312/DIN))
  (pad 1 smd rect (at -2.45 -1.6 135) (size 1.5 1) (layers F.Cu F.Paste F.Mask) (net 1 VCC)))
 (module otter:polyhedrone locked (layer F.Cu) (at 1.2 1.2)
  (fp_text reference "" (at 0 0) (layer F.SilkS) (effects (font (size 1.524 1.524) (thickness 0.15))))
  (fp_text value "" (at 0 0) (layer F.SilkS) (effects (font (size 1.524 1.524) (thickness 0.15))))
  (fp_line (start -1.12776 -1.12776) (end 2.46888 17.21612) (layer Edge.Cuts) (width 0.254))
  (fp_line (start 2.46888 17.21612) (end -0.25654 17.7546) (layer Edge.Cuts) (width 0.254))
  (fp_line (start -0.25654 17.7546) (end 1.54432 26.92654) (layer Edge.Cuts) (width 0.254))
  (fp_line (start 1.54432 26.92654) (end 7.00278 25.84958) (layer Edge.Cuts) (width 0.254))
  (fp_line (start 7.00278 25.84958) (end 7.2771 27.22626) (layer Edge.Cuts) (width 0.254))
  (fp_line (start 7.2771 27.22626) (end 6.36778 27.41168) (layer Edge.Cuts) (width 0.254))
  (fp_line (start 6.36778 27.41168) (end 7.62762 33.83026) (layer Edge.Cuts) (width 0.254))
  (fp_line (start 7.62762 33.83026) (end 8.53694 33.64738) (layer Edge.Cuts) (width 0.254))
  (fp_line (start 8.53694 33.64738) (end 8.8011 35.02152) (layer Edge.Cuts) (width 0.254))
  (fp_line (start 8.8011 35.02152) (end 6.07568 35.56) (layer Edge.Cuts) (width 0.254))
  (fp_line (start 6.07568 35.56) (end 9.67486 53.90388) (layer Edge.Cuts) (width 0.254))
  (fp_line (start 9.67486 53.90388) (end 6.94944 54.44236) (layer Edge.Cuts) (width 0.254))
  (fp_line (start 6.94944 54.44236) (end 8.74776 63.6143) (layer Edge.Cuts) (width 0.254))
  (fp_line (start 8.74776 63.6143) (end 14.20876 62.5475) (layer Edge.Cuts) (width 0.254))
  (fp_line (start 14.20876 62.5475) (end 14.48054 63.92418) (layer Edge.Cuts) (width 0.254))
  (fp_line (start 14.48054 63.92418) (end 13.57376 64.09944) (layer Edge.Cuts) (width 0.254))
  (fp_line (start 13.57376 64.09944) (end 14.82598 70.52056) (layer Edge.Cuts) (width 0.254))
  (fp_line (start 14.82598 70.52056) (end 15.74292 70.34276) (layer Edge.Cuts) (width 0.254))
  (fp_line (start 15.74292 70.34276) (end 16.00708 71.71944) (layer Edge.Cuts) (width 0.254))
  (fp_line (start 16.00708 71.71944) (end 13.28166 72.24776) (layer Edge.Cuts) (width 0.254))
  (fp_line (start 13.28166 72.24776) (end 16.88084 90.59418) (layer Edge.Cuts) (width 0.254))
  (fp_line (start 16.88084 90.59418) (end 25.29332 88.47582) (layer Edge.Cuts) (width 0.254))
  (fp_line (start 25.29332 88.47582) (end 25.97404 91.17584) (layer Edge.Cuts) (width 0.254))
  (fp_line (start 25.97404 91.17584) (end 34.38652 89.06002) (layer Edge.Cuts) (width 0.254))
  (fp_line (start 34.38652 89.06002) (end 33.02762 83.66252) (layer Edge.Cuts) (width 0.254))
  (fp_line (start 33.02762 83.66252) (end 34.29 83.34502) (layer Edge.Cuts) (width 0.254))
  (fp_line (start 34.29 83.34502) (end 34.5186 84.24418) (layer Edge.Cuts) (width 0.254))
  (fp_line (start 34.5186 84.24418) (end 40.40124 82.76082) (layer Edge.Cuts) (width 0.254))
  (fp_line (start 40.40124 82.76082) (end 40.18026 81.86166) (layer Edge.Cuts) (width 0.254))
  (fp_line (start 40.18026 81.86166) (end 41.44264 81.54416) (layer Edge.Cuts) (width 0.254))
  (fp_line (start 41.44264 81.54416) (end 42.12082 84.24418) (layer Edge.Cuts) (width 0.254))
  (fp_line (start 42.12082 84.24418) (end 50.53584 82.12582) (layer Edge.Cuts) (width 0.254))
  (fp_line (start 50.53584 82.12582) (end 51.21402 84.82584) (layer Edge.Cuts) (width 0.254))
  (fp_line (start 51.21402 84.82584) (end 59.61888 82.69986) (layer Edge.Cuts) (width 0.254))
  (fp_line (start 59.61888 82.69986) (end 58.26252 77.30236) (layer Edge.Cuts) (width 0.254))
  (fp_line (start 58.26252 77.30236) (end 59.52236 76.98486) (layer Edge.Cuts) (width 0.254))
  (fp_line (start 59.52236 76.98486) (end 59.75096 77.88402) (layer Edge.Cuts) (width 0.254))
  (fp_line (start 59.75096 77.88402) (end 65.64376 76.4032) (layer Edge.Cuts) (width 0.254))
  (fp_line (start 65.64376 76.4032) (end 65.41262 75.50404) (layer Edge.Cuts) (width 0.254))
  (fp_line (start 65.41262 75.50404) (end 66.675 75.18654) (layer Edge.Cuts) (width 0.254))
  (fp_line (start 66.675 75.18654) (end 67.35318 77.88402) (layer Edge.Cuts) (width 0.254))
  (fp_line (start 67.35318 77.88402) (end 75.7682 75.7682) (layer Edge.Cuts) (width 0.254))
  (fp_line (start 75.7682 75.7682) (end 77.88402 67.35318) (layer Edge.Cuts) (width 0.254))
  (fp_line (start 77.88402 67.35318) (end 80.58404 68.0339) (layer Edge.Cuts) (width 0.254))
  (fp_line (start 80.58404 68.0339) (end 82.69986 59.61888) (layer Edge.Cuts) (width 0.254))
  (fp_line (start 82.69986 59.61888) (end 77.30236 58.26252) (layer Edge.Cuts) (width 0.254))
  (fp_line (start 77.30236 58.26252) (end 77.63002 57.00014) (layer Edge.Cuts) (width 0.254))
  (fp_line (start 77.63002 57.00014) (end 78.52918 57.22874) (layer Edge.Cuts) (width 0.254))
  (fp_line (start 78.52918 57.22874) (end 80.01 51.33848) (layer Edge.Cuts) (width 0.254))
  (fp_line (start 80.01 51.33848) (end 79.11084 51.1175) (layer Edge.Cuts) (width 0.254))
  (fp_line (start 79.11084 51.1175) (end 79.42834 49.8475) (layer Edge.Cuts) (width 0.254))
  (fp_line (start 79.42834 49.8475) (end 82.12582 50.53584) (layer Edge.Cuts) (width 0.254))
  (fp_line (start 82.12582 50.53584) (end 84.24418 42.12082) (layer Edge.Cuts) (width 0.254))
  (fp_line (start 84.24418 42.12082) (end 86.94166 42.80154) (layer Edge.Cuts) (width 0.254))
  (fp_line (start 86.94166 42.80154) (end 89.06002 34.38652) (layer Edge.Cuts) (width 0.254))
  (fp_line (start 89.06002 34.38652) (end 83.66252 33.02762) (layer Edge.Cuts) (width 0.254))
  (fp_line (start 83.66252 33.02762) (end 83.98002 31.76778) (layer Edge.Cuts) (width 0.254))
  (fp_line (start 83.98002 31.76778) (end 84.87918 31.98876) (layer Edge.Cuts) (width 0.254))
  (fp_line (start 84.87918 31.98876) (end 86.36 26.10612) (layer Edge.Cuts) (width 0.254))
  (fp_line (start 86.36 26.10612) (end 85.46084 25.87752) (layer Edge.Cuts) (width 0.254))
  (fp_line (start 85.46084 25.87752) (end 85.77834 24.61514) (layer Edge.Cuts) (width 0.254))
  (fp_line (start 85.77834 24.61514) (end 88.47582 25.29332) (layer Edge.Cuts) (width 0.254))
  (fp_line (start 88.47582 25.29332) (end 90.59418 16.88084) (layer Edge.Cuts) (width 0.254))
  (fp_line (start 90.59418 16.88084) (end 72.24776 13.28166) (layer Edge.Cuts) (width 0.254))
  (fp_line (start 72.24776 13.28166) (end 72.78624 10.54862) (layer Edge.Cuts) (width 0.254))
  (fp_line (start 72.78624 10.54862) (end 63.6143 8.74776) (layer Edge.Cuts) (width 0.254))
  (fp_line (start 63.6143 8.74776) (end 62.5475 14.20876) (layer Edge.Cuts) (width 0.254))
  (fp_line (start 62.5475 14.20876) (end 61.17082 13.93444) (layer Edge.Cuts) (width 0.254))
  (fp_line (start 61.17082 13.93444) (end 61.34862 13.02512) (layer Edge.Cuts) (width 0.254))
  (fp_line (start 61.34862 13.02512) (end 54.9275 11.76528) (layer Edge.Cuts) (width 0.254))
  (fp_line (start 54.9275 11.76528) (end 54.74208 12.68222) (layer Edge.Cuts) (width 0.254))
  (fp_line (start 54.74208 12.68222) (end 53.3654 12.4079) (layer Edge.Cuts) (width 0.254))
  (fp_line (start 53.3654 12.4079) (end 53.90388 9.67486) (layer Edge.Cuts) (width 0.254))
  (fp_line (start 53.90388 9.67486) (end 35.56 6.07568) (layer Edge.Cuts) (width 0.254))
  (fp_line (start 35.56 6.07568) (end 36.09848 3.34264) (layer Edge.Cuts) (width 0.254))
  (fp_line (start 36.09848 3.34264) (end 26.92654 1.54432) (layer Edge.Cuts) (width 0.254))
  (fp_line (start 26.92654 1.54432) (end 25.84958 7.00278) (layer Edge.Cuts) (width 0.254))
  (fp_line (start 25.84958 7.00278) (end 24.4729 6.73862) (layer Edge.Cuts) (width 0.254))
  (fp_line (start 24.4729 6.73862) (end 24.65832 5.82168) (layer Edge.Cuts) (width 0.254))
  (fp_line (start 24.65832 5.82168) (end 18.23974 4.5593) (layer Edge.Cuts) (width 0.254))
  (fp_line (start 18.23974 4.5593) (end 18.05432 5.47624) (layer Edge.Cuts) (width 0.254))
  (fp_line (start 18.05432 5.47624) (end 16.67764 5.20446) (layer Edge.Cuts) (width 0.254))
  (fp_line (start 16.67764 5.20446) (end 17.21612 2.46888) (layer Edge.Cuts) (width 0.254))
  (fp_line (start 17.21612 2.46888) (end -1.12776 -1.12776) (layer Edge.Cuts) (width 0.254))
  (fp_line (start -1.12776 -1.12776) (end -1.12776 -1.12776) (layer Edge.Cuts) (width 0.254))
  (fp_line (start 42.3164 10.45972) (end 45.99432 11.17346) (layer Edge.Cuts) (width 0.254))
  (fp_line (start 45.99432 11.17346) (end 45.76318 12.3571) (layer Edge.Cuts) (width 0.254))
  (fp_line (start 45.76318 12.3571) (end 42.08526 11.64082) (layer Edge.Cuts) (width 0.254))
  (fp_line (start 42.08526 11.64082) (end 42.3164 10.45972) (layer Edge.Cuts) (width 0.254))
  (fp_line (start 42.3164 10.45972) (end 42.3164 10.45972) (layer Edge.Cuts) (width 0.254))
  (fp_line (start 11.6332 42.08526) (end 12.3571 45.75556) (layer Edge.Cuts) (width 0.254))
  (fp_line (start 12.3571 45.75556) (end 11.18362 45.98416) (layer Edge.Cuts) (width 0.254))
  (fp_line (start 11.18362 45.98416) (end 10.45972 42.32402) (layer Edge.Cuts) (width 0.254))
  (fp_line (start 10.45972 42.32402) (end 11.6332 42.08526) (layer Edge.Cuts) (width 0.254))
  (fp_line (start 11.6332 42.08526) (end 11.6332 42.08526) (layer Edge.Cuts) (width 0.254))
  (fp_line (start 79.53502 43.62196) (end 80.69834 43.91152) (layer Edge.Cuts) (width 0.254))
  (fp_line (start 80.69834 43.91152) (end 79.85252 47.2821) (layer Edge.Cuts) (width 0.254))
  (fp_line (start 79.85252 47.2821) (end 78.68666 46.98238) (layer Edge.Cuts) (width 0.254))
  (fp_line (start 78.68666 46.98238) (end 79.53502 43.62196) (layer Edge.Cuts) (width 0.254))
  (fp_line (start 79.53502 43.62196) (end 79.53502 43.62196) (layer Edge.Cuts) (width 0.254))
  (fp_line (start 46.98238 78.68666) (end 47.27194 79.85252) (layer Edge.Cuts) (width 0.254))
  (fp_line (start 47.27194 79.85252) (end 43.91152 80.69834) (layer Edge.Cuts) (width 0.254))
  (fp_line (start 43.91152 80.69834) (end 43.6118 79.53502) (layer Edge.Cuts) (width 0.254))
  (fp_line (start 43.6118 79.53502) (end 46.98238 78.68666) (layer Edge.Cuts) (width 0.254))
  (fp_line (start 46.98238 78.68666) (end 46.98238 78.68666) (layer Edge.Cuts) (width 0.254)))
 (segment (start 65.229696 31.550556) (end 65.777359 31.002893) (width 4) (layer B.Cu) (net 1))
 (segment (start 65.229696 38.885426) (end 65.229696 31.550556) (width 4) (layer B.Cu) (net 1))
 (segment (start 48.867107 60.787359) (end 32.374466 77.28) (width 4) (layer B.Cu) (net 8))
 (segment (start 32.374466 77.28) (end 29.03 77.28) (width 4) (layer B.Cu) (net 8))
 (segment (start 29.03 77.28) (end 23.62 77.28) (width 4) (layer B.Cu) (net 8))
 (segment (start 51.087561 58.566905) (end 48.867107 60.787359) (width 4) (layer B.Cu) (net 8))
 (segment (start 51.087561 53.027561) (end 51.087561 58.566905) (width 4) (layer B.Cu) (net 8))
 (segment (start 48.867107 60.787359) (end 61.154466 48.5) (width 4) (layer B.Cu) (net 8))
 (segment (start 61.154466 48.5) (end 63.88 48.5) (width 4) (layer B.Cu) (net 8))
 (segment (start 63.88 48.5) (end 75.7 36.68) (width 4) (layer B.Cu) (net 8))
 (segment (start 75.7 36.68) (end 75.7 25.37) (width 4) (layer B.Cu) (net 8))
 (segment (start 75.7 25.37) (end 76.96 24.11) (width 4) (layer B.Cu) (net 8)))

